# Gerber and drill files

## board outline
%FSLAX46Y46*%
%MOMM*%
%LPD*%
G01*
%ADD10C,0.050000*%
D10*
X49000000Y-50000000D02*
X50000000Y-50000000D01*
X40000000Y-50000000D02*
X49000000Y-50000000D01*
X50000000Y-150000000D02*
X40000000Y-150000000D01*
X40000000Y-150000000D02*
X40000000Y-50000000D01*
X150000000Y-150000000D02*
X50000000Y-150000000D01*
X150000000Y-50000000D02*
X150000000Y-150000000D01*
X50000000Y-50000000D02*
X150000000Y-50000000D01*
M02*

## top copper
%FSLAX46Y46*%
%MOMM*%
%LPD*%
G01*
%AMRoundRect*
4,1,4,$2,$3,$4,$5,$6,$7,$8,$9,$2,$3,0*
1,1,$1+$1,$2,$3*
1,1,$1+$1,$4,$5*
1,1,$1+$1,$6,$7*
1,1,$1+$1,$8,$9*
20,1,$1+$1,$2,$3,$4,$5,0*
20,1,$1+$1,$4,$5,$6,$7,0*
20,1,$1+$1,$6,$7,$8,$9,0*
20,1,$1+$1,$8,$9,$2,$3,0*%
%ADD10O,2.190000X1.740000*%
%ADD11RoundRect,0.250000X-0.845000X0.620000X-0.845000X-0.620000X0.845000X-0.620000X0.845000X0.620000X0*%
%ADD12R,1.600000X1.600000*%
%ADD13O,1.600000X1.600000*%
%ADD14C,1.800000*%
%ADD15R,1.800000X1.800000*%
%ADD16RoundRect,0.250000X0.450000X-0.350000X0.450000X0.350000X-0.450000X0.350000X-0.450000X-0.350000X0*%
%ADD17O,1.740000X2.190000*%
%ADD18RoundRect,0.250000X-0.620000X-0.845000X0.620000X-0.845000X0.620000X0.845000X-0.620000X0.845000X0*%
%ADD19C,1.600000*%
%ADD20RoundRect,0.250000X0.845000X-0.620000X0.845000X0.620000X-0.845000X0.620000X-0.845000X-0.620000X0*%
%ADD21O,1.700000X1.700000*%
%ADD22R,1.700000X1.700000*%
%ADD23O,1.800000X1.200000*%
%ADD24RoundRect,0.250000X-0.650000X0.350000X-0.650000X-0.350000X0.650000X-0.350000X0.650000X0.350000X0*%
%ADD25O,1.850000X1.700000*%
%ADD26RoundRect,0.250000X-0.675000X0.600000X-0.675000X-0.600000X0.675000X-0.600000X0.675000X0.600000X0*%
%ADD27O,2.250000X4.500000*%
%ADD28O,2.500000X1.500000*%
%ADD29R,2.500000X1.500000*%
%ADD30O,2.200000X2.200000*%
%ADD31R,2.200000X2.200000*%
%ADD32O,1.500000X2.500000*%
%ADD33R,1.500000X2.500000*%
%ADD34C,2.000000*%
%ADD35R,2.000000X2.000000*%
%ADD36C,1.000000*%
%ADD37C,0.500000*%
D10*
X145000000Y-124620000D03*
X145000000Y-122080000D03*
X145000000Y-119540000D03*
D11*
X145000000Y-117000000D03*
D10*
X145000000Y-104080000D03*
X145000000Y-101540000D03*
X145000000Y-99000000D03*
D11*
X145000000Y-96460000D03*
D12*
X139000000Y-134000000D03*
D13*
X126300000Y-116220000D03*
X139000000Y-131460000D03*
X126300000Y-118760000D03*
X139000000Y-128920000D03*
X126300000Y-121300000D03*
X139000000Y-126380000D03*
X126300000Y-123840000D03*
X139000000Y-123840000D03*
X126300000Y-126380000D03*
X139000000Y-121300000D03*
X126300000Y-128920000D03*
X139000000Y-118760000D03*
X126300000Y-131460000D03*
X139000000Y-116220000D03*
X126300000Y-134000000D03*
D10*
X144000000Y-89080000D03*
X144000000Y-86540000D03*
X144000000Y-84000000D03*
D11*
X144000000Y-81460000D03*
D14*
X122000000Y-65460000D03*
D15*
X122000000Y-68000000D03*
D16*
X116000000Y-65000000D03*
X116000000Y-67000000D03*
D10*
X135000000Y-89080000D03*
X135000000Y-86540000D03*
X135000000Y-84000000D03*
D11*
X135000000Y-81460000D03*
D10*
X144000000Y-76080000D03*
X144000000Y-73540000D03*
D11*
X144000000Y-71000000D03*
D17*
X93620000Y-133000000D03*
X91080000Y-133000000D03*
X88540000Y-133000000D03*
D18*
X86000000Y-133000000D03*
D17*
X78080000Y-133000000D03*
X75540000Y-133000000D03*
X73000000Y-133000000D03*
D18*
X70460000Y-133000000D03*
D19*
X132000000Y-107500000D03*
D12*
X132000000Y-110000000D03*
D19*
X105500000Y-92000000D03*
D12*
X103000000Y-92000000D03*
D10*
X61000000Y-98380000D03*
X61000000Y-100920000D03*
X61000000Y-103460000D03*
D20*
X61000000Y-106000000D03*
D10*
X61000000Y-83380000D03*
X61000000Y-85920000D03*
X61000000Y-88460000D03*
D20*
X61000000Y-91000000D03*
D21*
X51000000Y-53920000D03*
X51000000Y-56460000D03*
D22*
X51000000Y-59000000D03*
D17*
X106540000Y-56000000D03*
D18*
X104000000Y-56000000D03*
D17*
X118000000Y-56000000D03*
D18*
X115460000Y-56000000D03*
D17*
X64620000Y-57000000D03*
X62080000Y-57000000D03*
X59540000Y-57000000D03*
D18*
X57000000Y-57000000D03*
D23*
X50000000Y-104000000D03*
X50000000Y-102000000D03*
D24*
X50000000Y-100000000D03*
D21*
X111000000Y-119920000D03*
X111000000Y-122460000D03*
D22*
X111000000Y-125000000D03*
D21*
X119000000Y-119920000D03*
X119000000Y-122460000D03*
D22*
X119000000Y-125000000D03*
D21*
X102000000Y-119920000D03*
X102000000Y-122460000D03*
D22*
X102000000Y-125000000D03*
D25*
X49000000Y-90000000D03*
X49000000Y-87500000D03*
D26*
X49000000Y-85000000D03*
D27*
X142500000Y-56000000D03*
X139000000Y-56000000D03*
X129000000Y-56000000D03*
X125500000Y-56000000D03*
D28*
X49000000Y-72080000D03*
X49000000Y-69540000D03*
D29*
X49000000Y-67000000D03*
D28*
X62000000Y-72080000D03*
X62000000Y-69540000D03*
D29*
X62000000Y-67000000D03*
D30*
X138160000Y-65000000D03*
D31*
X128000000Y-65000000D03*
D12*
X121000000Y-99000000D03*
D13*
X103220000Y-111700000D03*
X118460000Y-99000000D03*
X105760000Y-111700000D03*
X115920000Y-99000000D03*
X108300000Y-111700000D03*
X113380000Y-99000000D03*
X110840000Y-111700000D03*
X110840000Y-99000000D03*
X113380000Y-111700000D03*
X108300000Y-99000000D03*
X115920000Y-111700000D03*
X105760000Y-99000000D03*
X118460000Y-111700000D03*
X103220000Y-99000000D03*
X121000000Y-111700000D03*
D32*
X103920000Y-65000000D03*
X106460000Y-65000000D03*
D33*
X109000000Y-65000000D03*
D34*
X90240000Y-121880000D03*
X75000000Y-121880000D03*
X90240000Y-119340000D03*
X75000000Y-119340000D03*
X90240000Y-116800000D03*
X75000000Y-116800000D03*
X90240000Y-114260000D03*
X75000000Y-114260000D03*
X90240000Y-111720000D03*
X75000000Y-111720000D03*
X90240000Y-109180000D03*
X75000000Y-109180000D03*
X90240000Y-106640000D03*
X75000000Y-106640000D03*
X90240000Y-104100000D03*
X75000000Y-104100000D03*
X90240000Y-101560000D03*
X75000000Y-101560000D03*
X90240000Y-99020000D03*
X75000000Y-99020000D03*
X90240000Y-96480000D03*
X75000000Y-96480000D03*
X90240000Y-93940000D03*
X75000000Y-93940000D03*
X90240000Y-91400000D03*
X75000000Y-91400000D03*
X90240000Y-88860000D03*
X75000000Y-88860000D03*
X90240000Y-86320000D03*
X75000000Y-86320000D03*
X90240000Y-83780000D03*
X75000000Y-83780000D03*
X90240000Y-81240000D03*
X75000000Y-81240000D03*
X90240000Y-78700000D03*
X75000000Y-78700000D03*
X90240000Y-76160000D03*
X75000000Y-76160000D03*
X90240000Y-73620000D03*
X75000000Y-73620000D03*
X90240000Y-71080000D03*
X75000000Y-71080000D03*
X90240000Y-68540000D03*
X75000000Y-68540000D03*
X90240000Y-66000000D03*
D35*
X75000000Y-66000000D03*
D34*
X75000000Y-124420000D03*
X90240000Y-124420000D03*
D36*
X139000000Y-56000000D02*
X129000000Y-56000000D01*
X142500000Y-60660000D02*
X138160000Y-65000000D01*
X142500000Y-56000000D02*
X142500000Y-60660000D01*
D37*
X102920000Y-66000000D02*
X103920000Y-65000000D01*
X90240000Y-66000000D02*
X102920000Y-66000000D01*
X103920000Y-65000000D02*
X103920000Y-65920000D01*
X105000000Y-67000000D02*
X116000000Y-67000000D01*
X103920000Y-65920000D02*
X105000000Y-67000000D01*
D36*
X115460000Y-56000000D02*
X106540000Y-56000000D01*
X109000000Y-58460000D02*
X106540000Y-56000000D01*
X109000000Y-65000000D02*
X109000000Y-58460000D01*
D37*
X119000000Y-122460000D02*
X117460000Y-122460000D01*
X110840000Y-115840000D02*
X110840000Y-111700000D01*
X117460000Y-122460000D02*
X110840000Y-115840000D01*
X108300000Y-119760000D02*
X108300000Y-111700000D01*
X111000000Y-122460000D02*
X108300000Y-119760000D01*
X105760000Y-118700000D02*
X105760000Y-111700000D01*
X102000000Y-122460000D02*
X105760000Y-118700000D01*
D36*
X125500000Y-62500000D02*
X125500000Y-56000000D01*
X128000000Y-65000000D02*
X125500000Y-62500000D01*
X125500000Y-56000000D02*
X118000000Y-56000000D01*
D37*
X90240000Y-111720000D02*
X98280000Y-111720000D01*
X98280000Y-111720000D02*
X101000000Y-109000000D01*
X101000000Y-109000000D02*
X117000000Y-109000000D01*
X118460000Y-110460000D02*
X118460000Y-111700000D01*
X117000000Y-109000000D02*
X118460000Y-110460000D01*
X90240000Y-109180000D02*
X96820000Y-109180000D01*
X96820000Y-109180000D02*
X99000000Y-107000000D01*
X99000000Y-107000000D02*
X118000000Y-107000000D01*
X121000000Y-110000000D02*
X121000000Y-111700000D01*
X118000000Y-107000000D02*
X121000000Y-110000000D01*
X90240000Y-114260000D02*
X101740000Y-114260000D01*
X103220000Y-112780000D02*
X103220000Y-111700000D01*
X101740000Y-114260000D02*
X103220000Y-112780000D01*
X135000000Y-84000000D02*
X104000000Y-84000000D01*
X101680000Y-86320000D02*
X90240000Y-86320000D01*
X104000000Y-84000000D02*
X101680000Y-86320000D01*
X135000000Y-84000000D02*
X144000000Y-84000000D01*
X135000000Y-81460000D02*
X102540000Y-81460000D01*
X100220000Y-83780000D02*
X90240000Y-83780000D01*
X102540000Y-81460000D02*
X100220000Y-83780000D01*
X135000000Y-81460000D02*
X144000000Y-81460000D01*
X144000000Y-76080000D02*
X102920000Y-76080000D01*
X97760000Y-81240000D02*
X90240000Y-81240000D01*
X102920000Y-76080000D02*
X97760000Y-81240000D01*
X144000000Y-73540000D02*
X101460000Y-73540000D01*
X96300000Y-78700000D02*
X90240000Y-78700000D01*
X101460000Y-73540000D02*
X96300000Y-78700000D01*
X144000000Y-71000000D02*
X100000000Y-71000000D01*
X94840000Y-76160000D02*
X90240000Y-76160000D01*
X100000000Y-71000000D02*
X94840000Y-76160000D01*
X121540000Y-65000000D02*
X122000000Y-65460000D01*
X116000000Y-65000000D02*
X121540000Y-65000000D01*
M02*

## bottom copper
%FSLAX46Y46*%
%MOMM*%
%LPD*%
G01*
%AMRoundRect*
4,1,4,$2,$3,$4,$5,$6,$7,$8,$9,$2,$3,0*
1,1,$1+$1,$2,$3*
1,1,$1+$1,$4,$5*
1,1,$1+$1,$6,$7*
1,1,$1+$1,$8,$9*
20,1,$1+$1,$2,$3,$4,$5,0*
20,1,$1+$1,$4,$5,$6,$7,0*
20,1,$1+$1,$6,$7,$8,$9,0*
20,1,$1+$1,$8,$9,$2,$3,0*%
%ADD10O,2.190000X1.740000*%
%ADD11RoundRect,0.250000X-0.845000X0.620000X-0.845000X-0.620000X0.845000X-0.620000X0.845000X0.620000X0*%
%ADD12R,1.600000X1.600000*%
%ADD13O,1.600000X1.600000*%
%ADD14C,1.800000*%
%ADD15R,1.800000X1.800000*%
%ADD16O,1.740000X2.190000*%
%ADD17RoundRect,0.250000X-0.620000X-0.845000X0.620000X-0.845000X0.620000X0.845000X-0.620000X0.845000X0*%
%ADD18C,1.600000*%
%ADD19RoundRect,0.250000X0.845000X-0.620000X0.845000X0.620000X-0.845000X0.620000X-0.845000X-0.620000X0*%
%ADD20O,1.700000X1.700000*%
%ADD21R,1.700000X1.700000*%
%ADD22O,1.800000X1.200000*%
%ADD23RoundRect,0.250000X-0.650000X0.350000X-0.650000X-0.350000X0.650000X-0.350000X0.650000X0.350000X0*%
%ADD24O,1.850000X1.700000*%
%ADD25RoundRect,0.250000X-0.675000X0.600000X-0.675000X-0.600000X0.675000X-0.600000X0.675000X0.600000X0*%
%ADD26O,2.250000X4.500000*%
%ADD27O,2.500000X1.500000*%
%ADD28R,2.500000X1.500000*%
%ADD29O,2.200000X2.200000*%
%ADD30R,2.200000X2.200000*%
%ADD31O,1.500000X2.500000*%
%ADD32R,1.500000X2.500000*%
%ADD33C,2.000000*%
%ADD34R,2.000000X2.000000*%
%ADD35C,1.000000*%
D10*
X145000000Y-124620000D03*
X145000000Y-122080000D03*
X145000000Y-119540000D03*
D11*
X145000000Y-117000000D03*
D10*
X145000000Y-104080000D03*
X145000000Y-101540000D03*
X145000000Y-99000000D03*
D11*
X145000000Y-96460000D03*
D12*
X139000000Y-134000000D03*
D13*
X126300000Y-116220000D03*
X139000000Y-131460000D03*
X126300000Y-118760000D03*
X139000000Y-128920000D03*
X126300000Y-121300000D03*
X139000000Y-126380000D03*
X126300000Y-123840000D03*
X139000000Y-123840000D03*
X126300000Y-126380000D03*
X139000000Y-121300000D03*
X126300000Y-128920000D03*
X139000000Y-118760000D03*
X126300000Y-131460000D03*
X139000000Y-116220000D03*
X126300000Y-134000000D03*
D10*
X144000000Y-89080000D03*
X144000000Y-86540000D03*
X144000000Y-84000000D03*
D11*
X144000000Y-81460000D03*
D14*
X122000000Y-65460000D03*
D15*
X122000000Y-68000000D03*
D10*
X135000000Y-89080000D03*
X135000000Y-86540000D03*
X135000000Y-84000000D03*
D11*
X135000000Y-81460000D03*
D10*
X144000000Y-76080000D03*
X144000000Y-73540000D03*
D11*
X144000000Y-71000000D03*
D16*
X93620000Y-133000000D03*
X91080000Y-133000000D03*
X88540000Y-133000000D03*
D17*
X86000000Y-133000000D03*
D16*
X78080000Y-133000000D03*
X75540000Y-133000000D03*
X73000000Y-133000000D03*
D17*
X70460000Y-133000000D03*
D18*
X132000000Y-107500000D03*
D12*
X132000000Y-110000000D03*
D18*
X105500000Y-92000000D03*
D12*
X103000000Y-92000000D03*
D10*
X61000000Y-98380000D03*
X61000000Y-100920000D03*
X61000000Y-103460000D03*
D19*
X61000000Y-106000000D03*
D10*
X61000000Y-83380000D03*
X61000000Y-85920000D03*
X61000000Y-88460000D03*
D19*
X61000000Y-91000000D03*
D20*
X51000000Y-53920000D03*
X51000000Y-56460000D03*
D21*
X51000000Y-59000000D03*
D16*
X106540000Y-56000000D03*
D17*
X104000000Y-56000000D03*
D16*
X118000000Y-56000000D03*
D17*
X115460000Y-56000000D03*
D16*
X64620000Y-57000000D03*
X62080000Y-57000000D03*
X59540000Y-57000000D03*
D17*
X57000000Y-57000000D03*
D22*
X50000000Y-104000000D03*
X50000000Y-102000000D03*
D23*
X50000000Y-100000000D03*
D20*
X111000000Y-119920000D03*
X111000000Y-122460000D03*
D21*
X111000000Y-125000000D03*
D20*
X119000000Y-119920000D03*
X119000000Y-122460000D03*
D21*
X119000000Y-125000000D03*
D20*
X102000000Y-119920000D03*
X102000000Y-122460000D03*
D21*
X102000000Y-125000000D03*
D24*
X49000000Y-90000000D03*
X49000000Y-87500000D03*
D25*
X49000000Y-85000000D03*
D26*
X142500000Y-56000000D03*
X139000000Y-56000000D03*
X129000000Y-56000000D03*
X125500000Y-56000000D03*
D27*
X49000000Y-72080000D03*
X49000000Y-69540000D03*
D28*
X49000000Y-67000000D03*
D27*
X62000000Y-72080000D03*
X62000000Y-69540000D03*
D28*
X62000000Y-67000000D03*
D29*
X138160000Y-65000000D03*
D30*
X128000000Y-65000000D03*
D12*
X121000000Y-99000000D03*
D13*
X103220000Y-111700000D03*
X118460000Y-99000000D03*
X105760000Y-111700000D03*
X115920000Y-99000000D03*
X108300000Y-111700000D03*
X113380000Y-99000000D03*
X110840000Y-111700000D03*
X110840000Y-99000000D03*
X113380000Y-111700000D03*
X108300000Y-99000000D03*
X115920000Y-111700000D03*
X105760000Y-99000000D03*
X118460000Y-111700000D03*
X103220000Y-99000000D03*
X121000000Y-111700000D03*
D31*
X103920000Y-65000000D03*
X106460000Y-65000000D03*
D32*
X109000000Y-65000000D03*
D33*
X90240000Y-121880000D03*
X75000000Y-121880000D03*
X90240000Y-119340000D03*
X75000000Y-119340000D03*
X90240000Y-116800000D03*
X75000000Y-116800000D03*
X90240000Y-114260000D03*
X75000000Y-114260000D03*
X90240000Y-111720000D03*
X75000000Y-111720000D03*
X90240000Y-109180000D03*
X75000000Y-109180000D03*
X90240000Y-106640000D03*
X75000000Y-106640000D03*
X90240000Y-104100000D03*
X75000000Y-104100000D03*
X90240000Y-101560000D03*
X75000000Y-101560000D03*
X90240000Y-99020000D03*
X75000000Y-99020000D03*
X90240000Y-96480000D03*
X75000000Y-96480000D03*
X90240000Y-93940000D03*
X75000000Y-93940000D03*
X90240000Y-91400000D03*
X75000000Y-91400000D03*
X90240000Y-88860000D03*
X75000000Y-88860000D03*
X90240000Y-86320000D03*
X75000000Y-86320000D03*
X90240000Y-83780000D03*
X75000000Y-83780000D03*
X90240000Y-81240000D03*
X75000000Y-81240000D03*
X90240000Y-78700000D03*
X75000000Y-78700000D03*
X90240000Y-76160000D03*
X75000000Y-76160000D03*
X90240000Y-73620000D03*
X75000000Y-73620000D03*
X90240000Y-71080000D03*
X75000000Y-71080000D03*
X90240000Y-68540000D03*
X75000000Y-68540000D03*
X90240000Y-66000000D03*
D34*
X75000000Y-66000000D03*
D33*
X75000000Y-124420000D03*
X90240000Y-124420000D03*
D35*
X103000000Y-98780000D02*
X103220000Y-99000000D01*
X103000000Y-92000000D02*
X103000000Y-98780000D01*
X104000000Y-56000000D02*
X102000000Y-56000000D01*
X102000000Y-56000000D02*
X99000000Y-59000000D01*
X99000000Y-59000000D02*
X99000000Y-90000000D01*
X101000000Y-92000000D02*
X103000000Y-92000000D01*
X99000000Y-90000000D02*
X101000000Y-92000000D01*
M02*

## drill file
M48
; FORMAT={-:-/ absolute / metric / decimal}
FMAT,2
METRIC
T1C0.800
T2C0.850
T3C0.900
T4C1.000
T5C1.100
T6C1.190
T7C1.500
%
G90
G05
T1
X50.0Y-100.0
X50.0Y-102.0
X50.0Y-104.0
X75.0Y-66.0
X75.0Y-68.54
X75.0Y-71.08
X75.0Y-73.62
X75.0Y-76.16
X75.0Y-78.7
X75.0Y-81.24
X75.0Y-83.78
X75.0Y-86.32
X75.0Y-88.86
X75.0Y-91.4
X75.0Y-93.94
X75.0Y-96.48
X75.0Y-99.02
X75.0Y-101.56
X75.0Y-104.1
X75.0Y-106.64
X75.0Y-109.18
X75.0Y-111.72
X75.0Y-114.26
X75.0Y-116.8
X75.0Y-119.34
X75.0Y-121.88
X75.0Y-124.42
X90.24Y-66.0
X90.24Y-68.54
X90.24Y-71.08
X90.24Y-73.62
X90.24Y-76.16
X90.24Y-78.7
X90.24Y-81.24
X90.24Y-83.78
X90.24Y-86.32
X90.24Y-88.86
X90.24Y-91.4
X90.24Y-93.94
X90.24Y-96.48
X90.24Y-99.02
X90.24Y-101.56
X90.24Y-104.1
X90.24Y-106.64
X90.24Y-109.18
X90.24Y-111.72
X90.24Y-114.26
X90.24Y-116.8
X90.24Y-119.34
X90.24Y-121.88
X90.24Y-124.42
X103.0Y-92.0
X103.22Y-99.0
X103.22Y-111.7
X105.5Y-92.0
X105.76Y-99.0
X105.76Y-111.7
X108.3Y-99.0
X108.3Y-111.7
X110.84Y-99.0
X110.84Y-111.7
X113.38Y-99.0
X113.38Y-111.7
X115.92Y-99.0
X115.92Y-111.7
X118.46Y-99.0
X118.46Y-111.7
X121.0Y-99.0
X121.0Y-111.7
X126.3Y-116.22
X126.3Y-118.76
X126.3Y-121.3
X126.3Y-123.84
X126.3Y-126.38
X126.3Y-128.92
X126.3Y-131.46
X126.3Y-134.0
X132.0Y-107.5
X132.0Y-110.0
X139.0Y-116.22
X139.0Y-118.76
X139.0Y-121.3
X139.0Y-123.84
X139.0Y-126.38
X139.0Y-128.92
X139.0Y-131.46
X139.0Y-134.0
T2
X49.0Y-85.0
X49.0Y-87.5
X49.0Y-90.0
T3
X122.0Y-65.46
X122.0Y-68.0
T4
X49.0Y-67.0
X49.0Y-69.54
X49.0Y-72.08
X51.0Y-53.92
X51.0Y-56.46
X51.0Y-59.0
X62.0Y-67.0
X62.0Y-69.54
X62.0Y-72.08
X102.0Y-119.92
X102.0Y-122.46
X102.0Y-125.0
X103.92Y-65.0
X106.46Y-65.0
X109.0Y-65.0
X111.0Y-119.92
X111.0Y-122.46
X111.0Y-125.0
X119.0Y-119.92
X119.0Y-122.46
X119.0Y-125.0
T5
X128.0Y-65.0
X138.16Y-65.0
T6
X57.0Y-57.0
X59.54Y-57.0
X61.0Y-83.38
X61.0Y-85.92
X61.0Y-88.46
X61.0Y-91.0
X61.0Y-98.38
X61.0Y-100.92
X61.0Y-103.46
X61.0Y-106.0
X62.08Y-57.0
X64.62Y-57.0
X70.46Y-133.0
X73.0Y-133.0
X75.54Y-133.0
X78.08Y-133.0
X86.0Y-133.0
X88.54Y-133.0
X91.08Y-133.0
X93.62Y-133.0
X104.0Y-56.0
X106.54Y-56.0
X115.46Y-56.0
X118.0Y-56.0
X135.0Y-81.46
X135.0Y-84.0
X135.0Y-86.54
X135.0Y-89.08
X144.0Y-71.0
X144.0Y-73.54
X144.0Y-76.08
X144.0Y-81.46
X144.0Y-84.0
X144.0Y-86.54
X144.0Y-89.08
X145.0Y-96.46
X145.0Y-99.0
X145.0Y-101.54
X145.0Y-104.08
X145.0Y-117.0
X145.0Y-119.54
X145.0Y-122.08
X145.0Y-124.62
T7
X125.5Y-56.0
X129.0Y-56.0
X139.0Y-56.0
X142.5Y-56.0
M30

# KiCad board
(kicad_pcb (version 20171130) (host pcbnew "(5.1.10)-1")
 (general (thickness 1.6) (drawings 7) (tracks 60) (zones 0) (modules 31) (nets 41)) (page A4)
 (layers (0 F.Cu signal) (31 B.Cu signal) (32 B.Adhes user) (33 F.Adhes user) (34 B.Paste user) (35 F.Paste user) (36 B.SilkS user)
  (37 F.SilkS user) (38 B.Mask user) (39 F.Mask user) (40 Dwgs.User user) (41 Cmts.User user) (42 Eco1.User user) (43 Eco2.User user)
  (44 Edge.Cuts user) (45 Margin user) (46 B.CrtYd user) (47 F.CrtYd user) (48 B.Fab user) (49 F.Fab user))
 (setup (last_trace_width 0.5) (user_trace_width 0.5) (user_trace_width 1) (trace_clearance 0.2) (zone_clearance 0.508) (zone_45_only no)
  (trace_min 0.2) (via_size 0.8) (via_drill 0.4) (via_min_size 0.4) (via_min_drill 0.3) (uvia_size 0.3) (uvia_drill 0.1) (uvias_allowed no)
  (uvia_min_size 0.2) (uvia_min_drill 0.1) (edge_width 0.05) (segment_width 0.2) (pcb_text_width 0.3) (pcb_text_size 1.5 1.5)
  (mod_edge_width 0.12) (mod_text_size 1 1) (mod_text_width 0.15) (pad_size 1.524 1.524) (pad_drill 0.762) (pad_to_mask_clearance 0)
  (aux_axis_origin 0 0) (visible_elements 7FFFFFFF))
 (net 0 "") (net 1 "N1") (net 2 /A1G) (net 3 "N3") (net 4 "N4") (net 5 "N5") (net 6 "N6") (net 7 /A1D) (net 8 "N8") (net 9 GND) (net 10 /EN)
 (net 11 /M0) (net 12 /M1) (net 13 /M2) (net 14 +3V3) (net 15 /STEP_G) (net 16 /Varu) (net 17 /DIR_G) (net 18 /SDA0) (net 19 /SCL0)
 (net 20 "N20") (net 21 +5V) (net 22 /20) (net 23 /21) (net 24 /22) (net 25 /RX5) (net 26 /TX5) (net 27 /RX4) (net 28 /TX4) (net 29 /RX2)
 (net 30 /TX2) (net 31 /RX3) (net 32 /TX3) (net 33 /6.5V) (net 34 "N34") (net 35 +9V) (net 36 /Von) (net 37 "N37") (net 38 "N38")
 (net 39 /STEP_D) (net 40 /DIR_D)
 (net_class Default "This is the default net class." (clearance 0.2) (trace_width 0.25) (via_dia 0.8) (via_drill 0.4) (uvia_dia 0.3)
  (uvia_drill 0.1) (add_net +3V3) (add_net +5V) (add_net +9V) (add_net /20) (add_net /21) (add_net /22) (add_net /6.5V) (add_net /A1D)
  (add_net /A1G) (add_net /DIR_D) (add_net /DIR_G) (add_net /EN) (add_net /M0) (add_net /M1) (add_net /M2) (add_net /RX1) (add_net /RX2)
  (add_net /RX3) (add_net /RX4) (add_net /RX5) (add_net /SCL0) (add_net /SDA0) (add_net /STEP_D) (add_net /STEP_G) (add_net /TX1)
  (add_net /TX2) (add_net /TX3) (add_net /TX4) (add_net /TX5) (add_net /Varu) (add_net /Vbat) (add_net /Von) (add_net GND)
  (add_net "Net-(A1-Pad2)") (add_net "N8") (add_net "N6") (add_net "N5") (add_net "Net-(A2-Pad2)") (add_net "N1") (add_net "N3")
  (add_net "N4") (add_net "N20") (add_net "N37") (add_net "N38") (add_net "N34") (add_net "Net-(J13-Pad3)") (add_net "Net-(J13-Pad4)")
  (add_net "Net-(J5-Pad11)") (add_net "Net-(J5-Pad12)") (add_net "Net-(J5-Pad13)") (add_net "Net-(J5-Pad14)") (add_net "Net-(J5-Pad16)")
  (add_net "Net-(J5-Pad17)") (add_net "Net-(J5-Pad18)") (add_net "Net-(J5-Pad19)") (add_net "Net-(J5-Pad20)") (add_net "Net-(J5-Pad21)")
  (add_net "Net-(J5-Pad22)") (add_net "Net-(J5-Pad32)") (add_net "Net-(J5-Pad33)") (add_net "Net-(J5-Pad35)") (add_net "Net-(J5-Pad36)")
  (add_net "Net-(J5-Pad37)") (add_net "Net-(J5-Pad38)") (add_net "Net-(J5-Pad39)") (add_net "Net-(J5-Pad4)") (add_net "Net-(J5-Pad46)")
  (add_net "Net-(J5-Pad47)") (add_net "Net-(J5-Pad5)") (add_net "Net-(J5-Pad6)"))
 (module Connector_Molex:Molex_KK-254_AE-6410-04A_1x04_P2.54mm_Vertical (layer F.Cu) (at 145 117 270)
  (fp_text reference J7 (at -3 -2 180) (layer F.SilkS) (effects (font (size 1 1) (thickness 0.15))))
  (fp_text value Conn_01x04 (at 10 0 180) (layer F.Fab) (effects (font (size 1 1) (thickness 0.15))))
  (pad 4 thru_hole oval (at 7.62 0 270) (size 1.74 2.19) (drill 1.19) (layers *.Cu *.Mask) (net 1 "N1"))
  (pad 3 thru_hole oval (at 5.08 0 270) (size 1.74 2.19) (drill 1.19) (layers *.Cu *.Mask) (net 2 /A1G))
  (pad 2 thru_hole oval (at 2.54 0 270) (size 1.74 2.19) (drill 1.19) (layers *.Cu *.Mask) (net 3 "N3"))
  (pad 1 thru_hole roundrect (at 0 0 270) (size 1.74 2.19) (drill 1.19) (layers *.Cu *.Mask) (roundrect_rratio 0.143678) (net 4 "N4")))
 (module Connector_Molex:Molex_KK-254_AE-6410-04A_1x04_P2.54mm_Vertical (layer F.Cu) (at 145 96.46 270)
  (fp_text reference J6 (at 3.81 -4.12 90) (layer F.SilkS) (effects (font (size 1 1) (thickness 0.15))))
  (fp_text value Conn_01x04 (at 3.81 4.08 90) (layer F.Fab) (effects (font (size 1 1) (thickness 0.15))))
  (pad 4 thru_hole oval (at 7.62 0 270) (size 1.74 2.19) (drill 1.19) (layers *.Cu *.Mask) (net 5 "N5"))
  (pad 3 thru_hole oval (at 5.08 0 270) (size 1.74 2.19) (drill 1.19) (layers *.Cu *.Mask) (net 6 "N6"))
  (pad 2 thru_hole oval (at 2.54 0 270) (size 1.74 2.19) (drill 1.19) (layers *.Cu *.Mask) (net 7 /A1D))
  (pad 1 thru_hole roundrect (at 0 0 270) (size 1.74 2.19) (drill 1.19) (layers *.Cu *.Mask) (roundrect_rratio 0.143678) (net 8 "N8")))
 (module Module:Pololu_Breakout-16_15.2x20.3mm (layer F.Cu) (at 139 134 180)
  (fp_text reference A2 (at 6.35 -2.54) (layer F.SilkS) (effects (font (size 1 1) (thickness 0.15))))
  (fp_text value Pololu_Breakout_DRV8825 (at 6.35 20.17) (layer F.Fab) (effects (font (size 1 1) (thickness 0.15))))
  (pad 1 thru_hole rect (at 0 0 180) (size 1.6 1.6) (drill 0.8) (layers *.Cu *.Mask) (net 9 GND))
  (pad 9 thru_hole oval (at 12.7 17.78 180) (size 1.6 1.6) (drill 0.8) (layers *.Cu *.Mask) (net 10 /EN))
  (pad 2 thru_hole oval (at 0 2.54 180) (size 1.6 1.6) (drill 0.8) (layers *.Cu *.Mask))
  (pad 10 thru_hole oval (at 12.7 15.24 180) (size 1.6 1.6) (drill 0.8) (layers *.Cu *.Mask) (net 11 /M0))
  (pad 3 thru_hole oval (at 0 5.08 180) (size 1.6 1.6) (drill 0.8) (layers *.Cu *.Mask) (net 1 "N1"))
  (pad 11 thru_hole oval (at 12.7 12.7 180) (size 1.6 1.6) (drill 0.8) (layers *.Cu *.Mask) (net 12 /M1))
  (pad 4 thru_hole oval (at 0 7.62 180) (size 1.6 1.6) (drill 0.8) (layers *.Cu *.Mask) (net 2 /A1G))
  (pad 12 thru_hole oval (at 12.7 10.16 180) (size 1.6 1.6) (drill 0.8) (layers *.Cu *.Mask) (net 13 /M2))
  (pad 5 thru_hole oval (at 0 10.16 180) (size 1.6 1.6) (drill 0.8) (layers *.Cu *.Mask) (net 3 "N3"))
  (pad 13 thru_hole oval (at 12.7 7.62 180) (size 1.6 1.6) (drill 0.8) (layers *.Cu *.Mask) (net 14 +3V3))
  (pad 6 thru_hole oval (at 0 12.7 180) (size 1.6 1.6) (drill 0.8) (layers *.Cu *.Mask) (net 4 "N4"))
  (pad 14 thru_hole oval (at 12.7 5.08 180) (size 1.6 1.6) (drill 0.8) (layers *.Cu *.Mask) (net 14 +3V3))
  (pad 7 thru_hole oval (at 0 15.24 180) (size 1.6 1.6) (drill 0.8) (layers *.Cu *.Mask) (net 9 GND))
  (pad 15 thru_hole oval (at 12.7 2.54 180) (size 1.6 1.6) (drill 0.8) (layers *.Cu *.Mask) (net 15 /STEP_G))
  (pad 8 thru_hole oval (at 0 17.78 180) (size 1.6 1.6) (drill 0.8) (layers *.Cu *.Mask) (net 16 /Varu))
  (pad 16 thru_hole oval (at 12.7 0 180) (size 1.6 1.6) (drill 0.8) (layers *.Cu *.Mask) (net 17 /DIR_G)))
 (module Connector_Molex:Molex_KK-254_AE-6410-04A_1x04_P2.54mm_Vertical (layer F.Cu) (at 144 81.46 270)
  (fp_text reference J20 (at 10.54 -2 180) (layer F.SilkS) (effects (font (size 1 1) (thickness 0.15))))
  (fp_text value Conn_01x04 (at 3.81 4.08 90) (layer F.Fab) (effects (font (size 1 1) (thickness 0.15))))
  (pad 4 thru_hole oval (at 7.62 0 270) (size 1.74 2.19) (drill 1.19) (layers *.Cu *.Mask) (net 14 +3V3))
  (pad 3 thru_hole oval (at 5.08 0 270) (size 1.74 2.19) (drill 1.19) (layers *.Cu *.Mask) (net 9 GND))
  (pad 2 thru_hole oval (at 2.54 0 270) (size 1.74 2.19) (drill 1.19) (layers *.Cu *.Mask) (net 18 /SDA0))
  (pad 1 thru_hole roundrect (at 0 0 270) (size 1.74 2.19) (drill 1.19) (layers *.Cu *.Mask) (roundrect_rratio 0.143678) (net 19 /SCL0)))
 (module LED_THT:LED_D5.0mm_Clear (layer F.Cu) (at 122 68 90)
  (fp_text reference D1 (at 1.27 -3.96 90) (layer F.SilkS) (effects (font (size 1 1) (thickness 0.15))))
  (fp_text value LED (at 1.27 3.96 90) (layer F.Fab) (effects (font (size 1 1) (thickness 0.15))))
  (pad 2 thru_hole circle (at 2.54 0 90) (size 1.8 1.8) (drill 0.9) (layers *.Cu *.Mask) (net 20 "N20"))
  (pad 1 thru_hole rect (at 0 0 90) (size 1.8 1.8) (drill 0.9) (layers *.Cu *.Mask) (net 9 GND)))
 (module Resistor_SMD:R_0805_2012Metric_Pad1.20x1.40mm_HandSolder (layer F.Cu) (at 116 66 90)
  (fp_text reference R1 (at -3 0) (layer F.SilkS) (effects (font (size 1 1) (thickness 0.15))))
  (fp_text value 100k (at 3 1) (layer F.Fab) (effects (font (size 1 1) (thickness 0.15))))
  (pad 2 smd roundrect (at 1 0 90) (size 1.2 1.4) (layers F.Cu F.Paste F.Mask) (roundrect_rratio 0.208333) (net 20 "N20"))
  (pad 1 smd roundrect (at -1 0 90) (size 1.2 1.4) (layers F.Cu F.Paste F.Mask) (roundrect_rratio 0.208333) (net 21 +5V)))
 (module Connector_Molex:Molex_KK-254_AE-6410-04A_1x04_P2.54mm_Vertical (layer F.Cu) (at 135 81.46 270)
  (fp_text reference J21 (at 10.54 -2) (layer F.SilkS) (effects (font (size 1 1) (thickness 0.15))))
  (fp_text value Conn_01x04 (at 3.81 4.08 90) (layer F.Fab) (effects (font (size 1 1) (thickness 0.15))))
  (pad 4 thru_hole oval (at 7.62 0 270) (size 1.74 2.19) (drill 1.19) (layers *.Cu *.Mask) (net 14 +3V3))
  (pad 3 thru_hole oval (at 5.08 0 270) (size 1.74 2.19) (drill 1.19) (layers *.Cu *.Mask) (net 9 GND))
  (pad 2 thru_hole oval (at 2.54 0 270) (size 1.74 2.19) (drill 1.19) (layers *.Cu *.Mask) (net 18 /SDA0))
  (pad 1 thru_hole roundrect (at 0 0 270) (size 1.74 2.19) (drill 1.19) (layers *.Cu *.Mask) (roundrect_rratio 0.143678) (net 19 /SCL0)))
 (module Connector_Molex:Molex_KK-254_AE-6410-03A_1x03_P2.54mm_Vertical (layer F.Cu) (at 144 71 270)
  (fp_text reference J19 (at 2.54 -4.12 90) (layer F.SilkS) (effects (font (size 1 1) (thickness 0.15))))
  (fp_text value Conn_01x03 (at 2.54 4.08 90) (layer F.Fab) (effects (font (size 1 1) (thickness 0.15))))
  (pad 3 thru_hole oval (at 5.08 0 270) (size 1.74 2.19) (drill 1.19) (layers *.Cu *.Mask) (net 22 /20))
  (pad 2 thru_hole oval (at 2.54 0 270) (size 1.74 2.19) (drill 1.19) (layers *.Cu *.Mask) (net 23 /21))
  (pad 1 thru_hole roundrect (at 0 0 270) (size 1.74 2.19) (drill 1.19) (layers *.Cu *.Mask) (roundrect_rratio 0.143678) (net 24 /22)))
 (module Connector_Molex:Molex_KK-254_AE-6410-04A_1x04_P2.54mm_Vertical (layer F.Cu) (at 86 133)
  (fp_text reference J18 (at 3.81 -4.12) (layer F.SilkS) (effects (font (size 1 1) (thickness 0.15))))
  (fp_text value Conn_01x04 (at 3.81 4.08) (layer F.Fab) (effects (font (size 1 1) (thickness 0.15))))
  (pad 4 thru_hole oval (at 7.62 0) (size 1.74 2.19) (drill 1.19) (layers *.Cu *.Mask) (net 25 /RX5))
  (pad 3 thru_hole oval (at 5.08 0) (size 1.74 2.19) (drill 1.19) (layers *.Cu *.Mask) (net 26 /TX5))
  (pad 2 thru_hole oval (at 2.54 0) (size 1.74 2.19) (drill 1.19) (layers *.Cu *.Mask) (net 9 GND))
  (pad 1 thru_hole roundrect (at 0 0) (size 1.74 2.19) (drill 1.19) (layers *.Cu *.Mask) (roundrect_rratio 0.143678) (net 21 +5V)))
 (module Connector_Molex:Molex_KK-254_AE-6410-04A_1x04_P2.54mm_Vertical (layer F.Cu) (at 70.46 133)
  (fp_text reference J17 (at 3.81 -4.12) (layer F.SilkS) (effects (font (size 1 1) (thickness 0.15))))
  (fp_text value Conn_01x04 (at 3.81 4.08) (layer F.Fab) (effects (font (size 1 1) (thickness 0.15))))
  (pad 4 thru_hole oval (at 7.62 0) (size 1.74 2.19) (drill 1.19) (layers *.Cu *.Mask) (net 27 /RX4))
  (pad 3 thru_hole oval (at 5.08 0) (size 1.74 2.19) (drill 1.19) (layers *.Cu *.Mask) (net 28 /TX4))
  (pad 2 thru_hole oval (at 2.54 0) (size 1.74 2.19) (drill 1.19) (layers *.Cu *.Mask) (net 9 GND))
  (pad 1 thru_hole roundrect (at 0 0) (size 1.74 2.19) (drill 1.19) (layers *.Cu *.Mask) (roundrect_rratio 0.143678) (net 21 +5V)))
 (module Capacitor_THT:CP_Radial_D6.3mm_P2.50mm (layer F.Cu) (at 132 110 90)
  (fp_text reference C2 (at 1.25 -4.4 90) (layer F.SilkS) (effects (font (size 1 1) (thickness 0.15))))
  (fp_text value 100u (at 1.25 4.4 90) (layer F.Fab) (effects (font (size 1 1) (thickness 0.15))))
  (pad 2 thru_hole circle (at 2.5 0 90) (size 1.6 1.6) (drill 0.8) (layers *.Cu *.Mask) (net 9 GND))
  (pad 1 thru_hole rect (at 0 0 90) (size 1.6 1.6) (drill 0.8) (layers *.Cu *.Mask) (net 16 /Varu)))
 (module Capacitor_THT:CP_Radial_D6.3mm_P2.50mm (layer F.Cu) (at 103 92)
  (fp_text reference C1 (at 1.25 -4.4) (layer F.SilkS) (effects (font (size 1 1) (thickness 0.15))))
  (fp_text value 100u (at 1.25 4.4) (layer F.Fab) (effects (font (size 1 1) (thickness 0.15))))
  (pad 2 thru_hole circle (at 2.5 0) (size 1.6 1.6) (drill 0.8) (layers *.Cu *.Mask) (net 9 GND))
  (pad 1 thru_hole rect (at 0 0) (size 1.6 1.6) (drill 0.8) (layers *.Cu *.Mask) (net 16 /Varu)))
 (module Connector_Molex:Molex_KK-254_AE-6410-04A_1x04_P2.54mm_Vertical (layer F.Cu) (at 61 106 90)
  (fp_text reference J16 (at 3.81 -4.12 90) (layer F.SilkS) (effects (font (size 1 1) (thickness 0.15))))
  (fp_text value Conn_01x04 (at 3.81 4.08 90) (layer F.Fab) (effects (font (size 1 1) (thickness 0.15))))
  (pad 4 thru_hole oval (at 7.62 0 90) (size 1.74 2.19) (drill 1.19) (layers *.Cu *.Mask) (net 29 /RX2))
  (pad 3 thru_hole oval (at 5.08 0 90) (size 1.74 2.19) (drill 1.19) (layers *.Cu *.Mask) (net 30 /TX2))
  (pad 2 thru_hole oval (at 2.54 0 90) (size 1.74 2.19) (drill 1.19) (layers *.Cu *.Mask) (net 9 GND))
  (pad 1 thru_hole roundrect (at 0 0 90) (size 1.74 2.19) (drill 1.19) (layers *.Cu *.Mask) (roundrect_rratio 0.143678) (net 14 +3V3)))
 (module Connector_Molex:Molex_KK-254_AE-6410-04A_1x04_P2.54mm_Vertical (layer F.Cu) (at 61 91 90)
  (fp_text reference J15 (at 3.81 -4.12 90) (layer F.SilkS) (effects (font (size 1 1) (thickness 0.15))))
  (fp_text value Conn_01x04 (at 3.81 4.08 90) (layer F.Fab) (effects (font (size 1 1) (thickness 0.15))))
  (pad 4 thru_hole oval (at 7.62 0 90) (size 1.74 2.19) (drill 1.19) (layers *.Cu *.Mask) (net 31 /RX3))
  (pad 3 thru_hole oval (at 5.08 0 90) (size 1.74 2.19) (drill 1.19) (layers *.Cu *.Mask) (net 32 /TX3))
  (pad 2 thru_hole oval (at 2.54 0 90) (size 1.74 2.19) (drill 1.19) (layers *.Cu *.Mask) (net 9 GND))
  (pad 1 thru_hole roundrect (at 0 0 90) (size 1.74 2.19) (drill 1.19) (layers *.Cu *.Mask) (roundrect_rratio 0.143678) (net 14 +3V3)))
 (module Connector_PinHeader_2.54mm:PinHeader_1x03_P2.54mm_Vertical (layer F.Cu) (at 51 59 180)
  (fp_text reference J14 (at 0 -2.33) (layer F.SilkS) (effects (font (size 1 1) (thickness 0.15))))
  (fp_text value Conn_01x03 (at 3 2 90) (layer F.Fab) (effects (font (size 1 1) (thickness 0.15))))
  (pad 3 thru_hole oval (at 0 5.08 180) (size 1.7 1.7) (drill 1) (layers *.Cu *.Mask) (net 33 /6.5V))
  (pad 2 thru_hole oval (at 0 2.54 180) (size 1.7 1.7) (drill 1) (layers *.Cu *.Mask) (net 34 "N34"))
  (pad 1 thru_hole rect (at 0 0 180) (size 1.7 1.7) (drill 1) (layers *.Cu *.Mask) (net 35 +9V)))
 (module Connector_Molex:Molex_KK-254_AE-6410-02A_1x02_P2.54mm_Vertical (layer F.Cu) (at 104 56)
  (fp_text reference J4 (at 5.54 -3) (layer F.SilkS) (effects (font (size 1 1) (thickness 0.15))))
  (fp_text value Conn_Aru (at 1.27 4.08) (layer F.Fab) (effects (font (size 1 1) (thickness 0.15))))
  (pad 2 thru_hole oval (at 2.54 0) (size 1.74 2.19) (drill 1.19) (layers *.Cu *.Mask) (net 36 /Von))
  (pad 1 thru_hole roundrect (at 0 0) (size 1.74 2.19) (drill 1.19) (layers *.Cu *.Mask) (roundrect_rratio 0.143678) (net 16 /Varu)))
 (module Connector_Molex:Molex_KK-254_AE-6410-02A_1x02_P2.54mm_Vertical (layer F.Cu) (at 115.46 56)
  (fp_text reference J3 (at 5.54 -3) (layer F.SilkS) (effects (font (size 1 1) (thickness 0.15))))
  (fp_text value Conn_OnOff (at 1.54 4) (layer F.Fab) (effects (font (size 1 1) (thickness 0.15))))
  (pad 2 thru_hole oval (at 2.54 0) (size 1.74 2.19) (drill 1.19) (layers *.Cu *.Mask) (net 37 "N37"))
  (pad 1 thru_hole roundrect (at 0 0) (size 1.74 2.19) (drill 1.19) (layers *.Cu *.Mask) (roundrect_rratio 0.143678) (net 36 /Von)))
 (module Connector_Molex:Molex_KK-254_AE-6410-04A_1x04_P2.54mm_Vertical (layer F.Cu) (at 57 57)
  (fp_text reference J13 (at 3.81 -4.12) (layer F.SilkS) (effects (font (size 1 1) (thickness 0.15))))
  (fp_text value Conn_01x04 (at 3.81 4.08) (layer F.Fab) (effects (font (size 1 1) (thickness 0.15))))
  (pad 4 thru_hole oval (at 7.62 0) (size 1.74 2.19) (drill 1.19) (layers *.Cu *.Mask))
  (pad 3 thru_hole oval (at 5.08 0) (size 1.74 2.19) (drill 1.19) (layers *.Cu *.Mask))
  (pad 2 thru_hole oval (at 2.54 0) (size 1.74 2.19) (drill 1.19) (layers *.Cu *.Mask) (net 9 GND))
  (pad 1 thru_hole roundrect (at 0 0) (size 1.74 2.19) (drill 1.19) (layers *.Cu *.Mask) (roundrect_rratio 0.143678) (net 34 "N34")))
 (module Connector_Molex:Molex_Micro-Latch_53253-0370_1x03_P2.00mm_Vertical (layer F.Cu) (at 50 100 270)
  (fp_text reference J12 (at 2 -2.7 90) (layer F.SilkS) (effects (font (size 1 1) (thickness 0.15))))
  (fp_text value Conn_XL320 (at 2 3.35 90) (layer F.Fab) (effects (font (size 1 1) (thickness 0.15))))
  (pad 3 thru_hole oval (at 4 0 270) (size 1.2 1.8) (drill 0.8) (layers *.Cu *.Mask) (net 30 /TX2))
  (pad 2 thru_hole oval (at 2 0 270) (size 1.2 1.8) (drill 0.8) (layers *.Cu *.Mask) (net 33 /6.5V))
  (pad 1 thru_hole roundrect (at 0 0 270) (size 1.2 1.8) (drill 0.8) (layers *.Cu *.Mask) (roundrect_rratio 0.208333) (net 9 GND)))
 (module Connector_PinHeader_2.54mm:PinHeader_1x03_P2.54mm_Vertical (layer F.Cu) (at 111 125 180)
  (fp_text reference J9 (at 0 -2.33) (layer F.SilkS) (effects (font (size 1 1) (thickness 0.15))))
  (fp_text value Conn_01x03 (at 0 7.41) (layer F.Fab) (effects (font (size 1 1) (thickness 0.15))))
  (pad 3 thru_hole oval (at 0 5.08 180) (size 1.7 1.7) (drill 1) (layers *.Cu *.Mask) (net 9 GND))
  (pad 2 thru_hole oval (at 0 2.54 180) (size 1.7 1.7) (drill 1) (layers *.Cu *.Mask) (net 12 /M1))
  (pad 1 thru_hole rect (at 0 0 180) (size 1.7 1.7) (drill 1) (layers *.Cu *.Mask) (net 14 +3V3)))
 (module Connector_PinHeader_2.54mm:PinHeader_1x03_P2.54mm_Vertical (layer F.Cu) (at 119 125 180)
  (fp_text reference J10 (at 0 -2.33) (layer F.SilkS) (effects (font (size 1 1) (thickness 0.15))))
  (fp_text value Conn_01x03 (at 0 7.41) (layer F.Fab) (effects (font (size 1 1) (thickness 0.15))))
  (pad 3 thru_hole oval (at 0 5.08 180) (size 1.7 1.7) (drill 1) (layers *.Cu *.Mask) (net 9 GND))
  (pad 2 thru_hole oval (at 0 2.54 180) (size 1.7 1.7) (drill 1) (layers *.Cu *.Mask) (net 13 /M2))
  (pad 1 thru_hole rect (at 0 0 180) (size 1.7 1.7) (drill 1) (layers *.Cu *.Mask) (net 14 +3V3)))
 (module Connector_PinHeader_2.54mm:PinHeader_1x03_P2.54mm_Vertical (layer F.Cu) (at 102 125 180)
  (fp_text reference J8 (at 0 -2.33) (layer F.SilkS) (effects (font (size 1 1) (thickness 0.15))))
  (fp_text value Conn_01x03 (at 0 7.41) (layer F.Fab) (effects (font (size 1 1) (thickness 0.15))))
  (pad 3 thru_hole oval (at 0 5.08 180) (size 1.7 1.7) (drill 1) (layers *.Cu *.Mask) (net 9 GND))
  (pad 2 thru_hole oval (at 0 2.54 180) (size 1.7 1.7) (drill 1) (layers *.Cu *.Mask) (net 11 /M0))
  (pad 1 thru_hole rect (at 0 0 180) (size 1.7 1.7) (drill 1) (layers *.Cu *.Mask) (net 14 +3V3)))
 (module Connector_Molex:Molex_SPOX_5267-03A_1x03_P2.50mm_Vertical (layer F.Cu) (at 49 85 270)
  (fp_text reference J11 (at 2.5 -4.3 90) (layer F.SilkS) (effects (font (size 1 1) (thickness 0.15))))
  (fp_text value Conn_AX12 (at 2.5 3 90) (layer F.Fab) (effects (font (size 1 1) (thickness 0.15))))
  (pad 3 thru_hole oval (at 5 0 270) (size 1.7 1.85) (drill 0.85) (layers *.Cu *.Mask) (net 32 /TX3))
  (pad 2 thru_hole oval (at 2.5 0 270) (size 1.7 1.85) (drill 0.85) (layers *.Cu *.Mask) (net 35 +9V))
  (pad 1 thru_hole roundrect (at 0 0 270) (size 1.7 1.85) (drill 0.85) (layers *.Cu *.Mask) (roundrect_rratio 0.147059) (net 9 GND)))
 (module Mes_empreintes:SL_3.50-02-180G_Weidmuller (layer F.Cu) (at 139 56)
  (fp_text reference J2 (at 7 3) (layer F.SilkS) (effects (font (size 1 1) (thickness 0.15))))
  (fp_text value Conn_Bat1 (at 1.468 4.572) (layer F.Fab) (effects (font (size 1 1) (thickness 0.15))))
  (pad 2 thru_hole oval (at 3.5 0) (size 2.25 4.5) (drill 1.5) (layers *.Cu *.Mask) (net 9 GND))
  (pad 1 thru_hole oval (at 0 0) (size 2.25 4.5) (drill 1.5) (layers *.Cu *.Mask) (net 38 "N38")))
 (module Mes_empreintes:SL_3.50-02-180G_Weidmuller (layer F.Cu) (at 125.5 56)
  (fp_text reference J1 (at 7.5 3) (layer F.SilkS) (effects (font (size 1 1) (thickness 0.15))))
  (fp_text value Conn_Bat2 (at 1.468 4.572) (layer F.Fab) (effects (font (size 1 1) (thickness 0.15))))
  (pad 2 thru_hole oval (at 3.5 0) (size 2.25 4.5) (drill 1.5) (layers *.Cu *.Mask) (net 38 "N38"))
  (pad 1 thru_hole oval (at 0 0) (size 2.25 4.5) (drill 1.5) (layers *.Cu *.Mask) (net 37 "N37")))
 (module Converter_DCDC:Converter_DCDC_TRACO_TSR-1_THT (layer F.Cu) (at 49 67 270)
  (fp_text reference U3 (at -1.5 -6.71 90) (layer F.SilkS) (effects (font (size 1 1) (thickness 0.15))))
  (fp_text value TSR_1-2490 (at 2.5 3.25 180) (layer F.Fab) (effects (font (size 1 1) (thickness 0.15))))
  (pad 3 thru_hole oval (at 5.08 0 270) (size 1.5 2.5) (drill 1) (layers *.Cu *.Mask) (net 35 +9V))
  (pad 2 thru_hole oval (at 2.54 0 270) (size 1.5 2.5) (drill 1) (layers *.Cu *.Mask) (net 9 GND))
  (pad 1 thru_hole rect (at 0 0 270) (size 1.5 2.5) (drill 1) (layers *.Cu *.Mask) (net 16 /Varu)))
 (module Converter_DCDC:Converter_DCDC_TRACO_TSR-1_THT (layer F.Cu) (at 62 67 270)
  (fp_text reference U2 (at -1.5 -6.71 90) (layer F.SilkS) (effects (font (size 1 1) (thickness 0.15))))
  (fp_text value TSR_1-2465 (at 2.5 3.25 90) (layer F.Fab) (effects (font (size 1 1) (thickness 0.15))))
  (pad 3 thru_hole oval (at 5.08 0 270) (size 1.5 2.5) (drill 1) (layers *.Cu *.Mask) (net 33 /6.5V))
  (pad 2 thru_hole oval (at 2.54 0 270) (size 1.5 2.5) (drill 1) (layers *.Cu *.Mask) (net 9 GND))
  (pad 1 thru_hole rect (at 0 0 270) (size 1.5 2.5) (drill 1) (layers *.Cu *.Mask) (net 16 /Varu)))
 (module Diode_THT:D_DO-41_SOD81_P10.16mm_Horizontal (layer F.Cu) (at 128 65)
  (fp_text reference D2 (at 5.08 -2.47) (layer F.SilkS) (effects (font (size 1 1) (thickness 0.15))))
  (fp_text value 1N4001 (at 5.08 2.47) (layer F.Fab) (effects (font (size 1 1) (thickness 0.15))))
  (pad 2 thru_hole oval (at 10.16 0) (size 2.2 2.2) (drill 1.1) (layers *.Cu *.Mask) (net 9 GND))
  (pad 1 thru_hole rect (at 0 0) (size 2.2 2.2) (drill 1.1) (layers *.Cu *.Mask) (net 37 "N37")))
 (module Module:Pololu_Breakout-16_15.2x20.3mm (layer F.Cu) (at 121 99 270)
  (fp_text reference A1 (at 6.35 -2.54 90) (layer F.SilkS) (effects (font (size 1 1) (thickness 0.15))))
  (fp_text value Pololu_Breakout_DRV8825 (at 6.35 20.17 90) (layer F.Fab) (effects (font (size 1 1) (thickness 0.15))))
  (pad 1 thru_hole rect (at 0 0 270) (size 1.6 1.6) (drill 0.8) (layers *.Cu *.Mask) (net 9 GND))
  (pad 9 thru_hole oval (at 12.7 17.78 270) (size 1.6 1.6) (drill 0.8) (layers *.Cu *.Mask) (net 10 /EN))
  (pad 2 thru_hole oval (at 0 2.54 270) (size 1.6 1.6) (drill 0.8) (layers *.Cu *.Mask))
  (pad 10 thru_hole oval (at 12.7 15.24 270) (size 1.6 1.6) (drill 0.8) (layers *.Cu *.Mask) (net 11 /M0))
  (pad 3 thru_hole oval (at 0 5.08 270) (size 1.6 1.6) (drill 0.8) (layers *.Cu *.Mask) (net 8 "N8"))
  (pad 11 thru_hole oval (at 12.7 12.7 270) (size 1.6 1.6) (drill 0.8) (layers *.Cu *.Mask) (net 12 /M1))
  (pad 4 thru_hole oval (at 0 7.62 270) (size 1.6 1.6) (drill 0.8) (layers *.Cu *.Mask) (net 7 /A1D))
  (pad 12 thru_hole oval (at 12.7 10.16 270) (size 1.6 1.6) (drill 0.8) (layers *.Cu *.Mask) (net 13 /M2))
  (pad 5 thru_hole oval (at 0 10.16 270) (size 1.6 1.6) (drill 0.8) (layers *.Cu *.Mask) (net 6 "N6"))
  (pad 13 thru_hole oval (at 12.7 7.62 270) (size 1.6 1.6) (drill 0.8) (layers *.Cu *.Mask) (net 14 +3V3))
  (pad 6 thru_hole oval (at 0 12.7 270) (size 1.6 1.6) (drill 0.8) (layers *.Cu *.Mask) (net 5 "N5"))
  (pad 14 thru_hole oval (at 12.7 5.08 270) (size 1.6 1.6) (drill 0.8) (layers *.Cu *.Mask) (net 14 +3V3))
  (pad 7 thru_hole oval (at 0 15.24 270) (size 1.6 1.6) (drill 0.8) (layers *.Cu *.Mask) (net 9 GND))
  (pad 15 thru_hole oval (at 12.7 2.54 270) (size 1.6 1.6) (drill 0.8) (layers *.Cu *.Mask) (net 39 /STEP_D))
  (pad 8 thru_hole oval (at 0 17.78 270) (size 1.6 1.6) (drill 0.8) (layers *.Cu *.Mask) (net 16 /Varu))
  (pad 16 thru_hole oval (at 12.7 0 270) (size 1.6 1.6) (drill 0.8) (layers *.Cu *.Mask) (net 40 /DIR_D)))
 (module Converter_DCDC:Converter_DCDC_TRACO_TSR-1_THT (layer F.Cu) (at 109 65 180)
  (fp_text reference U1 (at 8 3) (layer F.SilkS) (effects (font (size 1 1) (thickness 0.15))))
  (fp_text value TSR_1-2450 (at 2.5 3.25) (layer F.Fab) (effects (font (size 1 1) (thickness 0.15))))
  (pad 3 thru_hole oval (at 5.08 0 180) (size 1.5 2.5) (drill 1) (layers *.Cu *.Mask) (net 21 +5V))
  (pad 2 thru_hole oval (at 2.54 0 180) (size 1.5 2.5) (drill 1) (layers *.Cu *.Mask) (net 9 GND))
  (pad 1 thru_hole rect (at 0 0 180) (size 1.5 2.5) (drill 1) (layers *.Cu *.Mask) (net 36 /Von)))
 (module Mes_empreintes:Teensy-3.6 (layer F.Cu) (at 75 66)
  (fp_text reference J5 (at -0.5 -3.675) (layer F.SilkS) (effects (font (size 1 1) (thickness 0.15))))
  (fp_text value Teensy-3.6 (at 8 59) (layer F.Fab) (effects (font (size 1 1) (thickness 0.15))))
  (pad 26 thru_hole circle (at 15.24 55.88) (size 2 2) (drill 0.8) (layers *.Cu *.Mask) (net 25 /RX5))
  (pad 23 thru_hole circle (at 0 55.88) (size 2 2) (drill 0.8) (layers *.Cu *.Mask) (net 27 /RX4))
  (pad 27 thru_hole circle (at 15.24 53.34) (size 2 2) (drill 0.8) (layers *.Cu *.Mask) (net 15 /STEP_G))
  (pad 22 thru_hole circle (at 0 53.34) (size 2 2) (drill 0.8) (layers *.Cu *.Mask))
  (pad 28 thru_hole circle (at 15.24 50.8) (size 2 2) (drill 0.8) (layers *.Cu *.Mask) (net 17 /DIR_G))
  (pad 21 thru_hole circle (at 0 50.8) (size 2 2) (drill 0.8) (layers *.Cu *.Mask))
  (pad 29 thru_hole circle (at 15.24 48.26) (size 2 2) (drill 0.8) (layers *.Cu *.Mask) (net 10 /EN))
  (pad 20 thru_hole circle (at 0 48.26) (size 2 2) (drill 0.8) (layers *.Cu *.Mask))
  (pad 30 thru_hole circle (at 15.24 45.72) (size 2 2) (drill 0.8) (layers *.Cu *.Mask) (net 39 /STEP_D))
  (pad 19 thru_hole circle (at 0 45.72) (size 2 2) (drill 0.8) (layers *.Cu *.Mask))
  (pad 31 thru_hole circle (at 15.24 43.18) (size 2 2) (drill 0.8) (layers *.Cu *.Mask) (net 40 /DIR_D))
  (pad 18 thru_hole circle (at 0 43.18) (size 2 2) (drill 0.8) (layers *.Cu *.Mask))
  (pad 32 thru_hole circle (at 15.24 40.64) (size 2 2) (drill 0.8) (layers *.Cu *.Mask))
  (pad 17 thru_hole circle (at 0 40.64) (size 2 2) (drill 0.8) (layers *.Cu *.Mask))
  (pad 33 thru_hole circle (at 15.24 38.1) (size 2 2) (drill 0.8) (layers *.Cu *.Mask))
  (pad 16 thru_hole circle (at 0 38.1) (size 2 2) (drill 0.8) (layers *.Cu *.Mask))
  (pad 34 thru_hole circle (at 15.24 35.56) (size 2 2) (drill 0.8) (layers *.Cu *.Mask) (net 9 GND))
  (pad 15 thru_hole circle (at 0 35.56) (size 2 2) (drill 0.8) (layers *.Cu *.Mask) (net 14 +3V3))
  (pad 35 thru_hole circle (at 15.24 33.02) (size 2 2) (drill 0.8) (layers *.Cu *.Mask))
  (pad 14 thru_hole circle (at 0 33.02) (size 2 2) (drill 0.8) (layers *.Cu *.Mask))
  (pad 36 thru_hole circle (at 15.24 30.48) (size 2 2) (drill 0.8) (layers *.Cu *.Mask))
  (pad 13 thru_hole circle (at 0 30.48) (size 2 2) (drill 0.8) (layers *.Cu *.Mask))
  (pad 37 thru_hole circle (at 15.24 27.94) (size 2 2) (drill 0.8) (layers *.Cu *.Mask))
  (pad 12 thru_hole circle (at 0 27.94) (size 2 2) (drill 0.8) (layers *.Cu *.Mask))
  (pad 38 thru_hole circle (at 15.24 25.4) (size 2 2) (drill 0.8) (layers *.Cu *.Mask))
  (pad 11 thru_hole circle (at 0 25.4) (size 2 2) (drill 0.8) (layers *.Cu *.Mask))
  (pad 39 thru_hole circle (at 15.24 22.86) (size 2 2) (drill 0.8) (layers *.Cu *.Mask))
  (pad 10 thru_hole circle (at 0 22.86) (size 2 2) (drill 0.8) (layers *.Cu *.Mask) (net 30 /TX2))
  (pad 40 thru_hole circle (at 15.24 20.32) (size 2 2) (drill 0.8) (layers *.Cu *.Mask) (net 18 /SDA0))
  (pad 9 thru_hole circle (at 0 20.32) (size 2 2) (drill 0.8) (layers *.Cu *.Mask) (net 29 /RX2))
  (pad 41 thru_hole circle (at 15.24 17.78) (size 2 2) (drill 0.8) (layers *.Cu *.Mask) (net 19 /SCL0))
  (pad 8 thru_hole circle (at 0 17.78) (size 2 2) (drill 0.8) (layers *.Cu *.Mask) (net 32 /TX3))
  (pad 42 thru_hole circle (at 15.24 15.24) (size 2 2) (drill 0.8) (layers *.Cu *.Mask) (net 22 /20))
  (pad 7 thru_hole circle (at 0 15.24) (size 2 2) (drill 0.8) (layers *.Cu *.Mask) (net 31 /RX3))
  (pad 43 thru_hole circle (at 15.24 12.7) (size 2 2) (drill 0.8) (layers *.Cu *.Mask) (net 23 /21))
  (pad 6 thru_hole circle (at 0 12.7) (size 2 2) (drill 0.8) (layers *.Cu *.Mask))
  (pad 44 thru_hole circle (at 15.24 10.16) (size 2 2) (drill 0.8) (layers *.Cu *.Mask) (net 24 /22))
  (pad 5 thru_hole circle (at 0 10.16) (size 2 2) (drill 0.8) (layers *.Cu *.Mask))
  (pad 45 thru_hole circle (at 15.24 7.62) (size 2 2) (drill 0.8) (layers *.Cu *.Mask))
  (pad 4 thru_hole circle (at 0 7.62) (size 2 2) (drill 0.8) (layers *.Cu *.Mask))
  (pad 46 thru_hole circle (at 15.24 5.08) (size 2 2) (drill 0.8) (layers *.Cu *.Mask))
  (pad 3 thru_hole circle (at 0 5.08) (size 2 2) (drill 0.8) (layers *.Cu *.Mask))
  (pad 47 thru_hole circle (at 15.24 2.54) (size 2 2) (drill 0.8) (layers *.Cu *.Mask))
  (pad 2 thru_hole circle (at 0 2.54) (size 2 2) (drill 0.8) (layers *.Cu *.Mask))
  (pad 48 thru_hole circle (at 15.24 0) (size 2 2) (drill 0.8) (layers *.Cu *.Mask) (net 21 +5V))
  (pad 1 thru_hole rect (at 0 0) (size 2 2) (drill 0.8) (layers *.Cu *.Mask) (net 9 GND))
  (pad 24 thru_hole circle (at 0 58.42) (size 2 2) (drill 0.8) (layers *.Cu *.Mask) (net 28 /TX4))
  (pad 25 thru_hole circle (at 15.24 58.42) (size 2 2) (drill 0.8) (layers *.Cu *.Mask) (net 26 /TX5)))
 (gr_line (start 49 50) (end 50 50) (layer Edge.Cuts) (width 0.05))
 (gr_line (start 40 50) (end 49 50) (layer Edge.Cuts) (width 0.05))
 (gr_line (start 50 150) (end 40 150) (layer Edge.Cuts) (width 0.05))
 (gr_line (start 40 150) (end 40 50) (layer Edge.Cuts) (width 0.05))
 (gr_line (start 150 150) (end 50 150) (layer Edge.Cuts) (width 0.05))
 (gr_line (start 150 50) (end 150 150) (layer Edge.Cuts) (width 0.05))
 (gr_line (start 50 50) (end 150 50) (layer Edge.Cuts) (width 0.05))
 (segment (start 139 56) (end 129 56) (width 1) (layer F.Cu) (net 38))
 (segment (start 142.5 60.66) (end 138.16 65) (width 1) (layer F.Cu) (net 9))
 (segment (start 142.5 56) (end 142.5 60.66) (width 1) (layer F.Cu) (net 9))
 (segment (start 102.92 66) (end 103.92 65) (width 0.5) (layer F.Cu) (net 21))
 (segment (start 90.24 66) (end 102.92 66) (width 0.5) (layer F.Cu) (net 21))
 (segment (start 103.92 65) (end 103.92 65.92) (width 0.5) (layer F.Cu) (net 21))
 (segment (start 105 67) (end 116 67) (width 0.5) (layer F.Cu) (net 21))
 (segment (start 103.92 65.92) (end 105 67) (width 0.5) (layer F.Cu) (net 21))
 (segment (start 115.46 56) (end 106.54 56) (width 1) (layer F.Cu) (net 36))
 (segment (start 109 58.46) (end 106.54 56) (width 1) (layer F.Cu) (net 36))
 (segment (start 109 65) (end 109 58.46) (width 1) (layer F.Cu) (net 36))
 (segment (start 119 122.46) (end 117.46 122.46) (width 0.5) (layer F.Cu) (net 13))
 (segment (start 110.84 115.84) (end 110.84 111.7) (width 0.5) (layer F.Cu) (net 13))
 (segment (start 117.46 122.46) (end 110.84 115.84) (width 0.5) (layer F.Cu) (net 13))
 (segment (start 108.3 119.76) (end 108.3 111.7) (width 0.5) (layer F.Cu) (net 12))
 (segment (start 111 122.46) (end 108.3 119.76) (width 0.5) (layer F.Cu) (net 12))
 (segment (start 105.76 118.7) (end 105.76 111.7) (width 0.5) (layer F.Cu) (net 11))
 (segment (start 102 122.46) (end 105.76 118.7) (width 0.5) (layer F.Cu) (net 11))
 (segment (start 125.5 62.5) (end 125.5 56) (width 1) (layer F.Cu) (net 37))
 (segment (start 128 65) (end 125.5 62.5) (width 1) (layer F.Cu) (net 37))
 (segment (start 125.5 56) (end 118 56) (width 1) (layer F.Cu) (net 37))
 (segment (start 90.24 111.72) (end 98.28 111.72) (width 0.5) (layer F.Cu) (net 39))
 (segment (start 98.28 111.72) (end 101 109) (width 0.5) (layer F.Cu) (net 39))
 (segment (start 101 109) (end 117 109) (width 0.5) (layer F.Cu) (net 39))
 (segment (start 118.46 110.46) (end 118.46 111.7) (width 0.5) (layer F.Cu) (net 39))
 (segment (start 117 109) (end 118.46 110.46) (width 0.5) (layer F.Cu) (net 39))
 (segment (start 103 98.78) (end 103.22 99) (width 1) (layer B.Cu) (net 16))
 (segment (start 103 92) (end 103 98.78) (width 1) (layer B.Cu) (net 16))
 (segment (start 104 56) (end 102 56) (width 1) (layer B.Cu) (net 16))
 (segment (start 102 56) (end 99 59) (width 1) (layer B.Cu) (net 16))
 (segment (start 99 59) (end 99 90) (width 1) (layer B.Cu) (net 16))
 (segment (start 101 92) (end 103 92) (width 1) (layer B.Cu) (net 16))
 (segment (start 99 90) (end 101 92) (width 1) (layer B.Cu) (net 16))
 (segment (start 90.24 109.18) (end 96.82 109.18) (width 0.5) (layer F.Cu) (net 40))
 (segment (start 96.82 109.18) (end 99 107) (width 0.5) (layer F.Cu) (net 40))
 (segment (start 99 107) (end 118 107) (width 0.5) (layer F.Cu) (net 40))
 (segment (start 121 110) (end 121 111.7) (width 0.5) (layer F.Cu) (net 40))
 (segment (start 118 107) (end 121 110) (width 0.5) (layer F.Cu) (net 40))
 (segment (start 90.24 114.26) (end 101.74 114.26) (width 0.5) (layer F.Cu) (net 10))
 (segment (start 103.22 112.78) (end 103.22 111.7) (width 0.5) (layer F.Cu) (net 10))
 (segment (start 101.74 114.26) (end 103.22 112.78) (width 0.5) (layer F.Cu) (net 10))
 (segment (start 135 84) (end 104 84) (width 0.5) (layer F.Cu) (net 18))
 (segment (start 101.68 86.32) (end 90.24 86.32) (width 0.5) (layer F.Cu) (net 18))
 (segment (start 104 84) (end 101.68 86.32) (width 0.5) (layer F.Cu) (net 18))
 (segment (start 135 84) (end 144 84) (width 0.5) (layer F.Cu) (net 18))
 (segment (start 135 81.46) (end 102.54 81.46) (width 0.5) (layer F.Cu) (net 19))
 (segment (start 100.22 83.78) (end 90.24 83.78) (width 0.5) (layer F.Cu) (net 19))
 (segment (start 102.54 81.46) (end 100.22 83.78) (width 0.5) (layer F.Cu) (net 19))
 (segment (start 135 81.46) (end 144 81.46) (width 0.5) (layer F.Cu) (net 19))
 (segment (start 144 76.08) (end 102.92 76.08) (width 0.5) (layer F.Cu) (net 22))
 (segment (start 97.76 81.24) (end 90.24 81.24) (width 0.5) (layer F.Cu) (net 22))
 (segment (start 102.92 76.08) (end 97.76 81.24) (width 0.5) (layer F.Cu) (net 22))
 (segment (start 144 73.54) (end 101.46 73.54) (width 0.5) (layer F.Cu) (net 23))
 (segment (start 96.3 78.7) (end 90.24 78.7) (width 0.5) (layer F.Cu) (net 23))
 (segment (start 101.46 73.54) (end 96.3 78.7) (width 0.5) (layer F.Cu) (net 23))
 (segment (start 144 71) (end 100 71) (width 0.5) (layer F.Cu) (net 24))
 (segment (start 94.84 76.16) (end 90.24 76.16) (width 0.5) (layer F.Cu) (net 24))
 (segment (start 100 71) (end 94.84 76.16) (width 0.5) (layer F.Cu) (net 24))
 (segment (start 121.54 65) (end 122 65.46) (width 0.5) (layer F.Cu) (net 20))
 (segment (start 116 65) (end 121.54 65) (width 0.5) (layer F.Cu) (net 20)))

